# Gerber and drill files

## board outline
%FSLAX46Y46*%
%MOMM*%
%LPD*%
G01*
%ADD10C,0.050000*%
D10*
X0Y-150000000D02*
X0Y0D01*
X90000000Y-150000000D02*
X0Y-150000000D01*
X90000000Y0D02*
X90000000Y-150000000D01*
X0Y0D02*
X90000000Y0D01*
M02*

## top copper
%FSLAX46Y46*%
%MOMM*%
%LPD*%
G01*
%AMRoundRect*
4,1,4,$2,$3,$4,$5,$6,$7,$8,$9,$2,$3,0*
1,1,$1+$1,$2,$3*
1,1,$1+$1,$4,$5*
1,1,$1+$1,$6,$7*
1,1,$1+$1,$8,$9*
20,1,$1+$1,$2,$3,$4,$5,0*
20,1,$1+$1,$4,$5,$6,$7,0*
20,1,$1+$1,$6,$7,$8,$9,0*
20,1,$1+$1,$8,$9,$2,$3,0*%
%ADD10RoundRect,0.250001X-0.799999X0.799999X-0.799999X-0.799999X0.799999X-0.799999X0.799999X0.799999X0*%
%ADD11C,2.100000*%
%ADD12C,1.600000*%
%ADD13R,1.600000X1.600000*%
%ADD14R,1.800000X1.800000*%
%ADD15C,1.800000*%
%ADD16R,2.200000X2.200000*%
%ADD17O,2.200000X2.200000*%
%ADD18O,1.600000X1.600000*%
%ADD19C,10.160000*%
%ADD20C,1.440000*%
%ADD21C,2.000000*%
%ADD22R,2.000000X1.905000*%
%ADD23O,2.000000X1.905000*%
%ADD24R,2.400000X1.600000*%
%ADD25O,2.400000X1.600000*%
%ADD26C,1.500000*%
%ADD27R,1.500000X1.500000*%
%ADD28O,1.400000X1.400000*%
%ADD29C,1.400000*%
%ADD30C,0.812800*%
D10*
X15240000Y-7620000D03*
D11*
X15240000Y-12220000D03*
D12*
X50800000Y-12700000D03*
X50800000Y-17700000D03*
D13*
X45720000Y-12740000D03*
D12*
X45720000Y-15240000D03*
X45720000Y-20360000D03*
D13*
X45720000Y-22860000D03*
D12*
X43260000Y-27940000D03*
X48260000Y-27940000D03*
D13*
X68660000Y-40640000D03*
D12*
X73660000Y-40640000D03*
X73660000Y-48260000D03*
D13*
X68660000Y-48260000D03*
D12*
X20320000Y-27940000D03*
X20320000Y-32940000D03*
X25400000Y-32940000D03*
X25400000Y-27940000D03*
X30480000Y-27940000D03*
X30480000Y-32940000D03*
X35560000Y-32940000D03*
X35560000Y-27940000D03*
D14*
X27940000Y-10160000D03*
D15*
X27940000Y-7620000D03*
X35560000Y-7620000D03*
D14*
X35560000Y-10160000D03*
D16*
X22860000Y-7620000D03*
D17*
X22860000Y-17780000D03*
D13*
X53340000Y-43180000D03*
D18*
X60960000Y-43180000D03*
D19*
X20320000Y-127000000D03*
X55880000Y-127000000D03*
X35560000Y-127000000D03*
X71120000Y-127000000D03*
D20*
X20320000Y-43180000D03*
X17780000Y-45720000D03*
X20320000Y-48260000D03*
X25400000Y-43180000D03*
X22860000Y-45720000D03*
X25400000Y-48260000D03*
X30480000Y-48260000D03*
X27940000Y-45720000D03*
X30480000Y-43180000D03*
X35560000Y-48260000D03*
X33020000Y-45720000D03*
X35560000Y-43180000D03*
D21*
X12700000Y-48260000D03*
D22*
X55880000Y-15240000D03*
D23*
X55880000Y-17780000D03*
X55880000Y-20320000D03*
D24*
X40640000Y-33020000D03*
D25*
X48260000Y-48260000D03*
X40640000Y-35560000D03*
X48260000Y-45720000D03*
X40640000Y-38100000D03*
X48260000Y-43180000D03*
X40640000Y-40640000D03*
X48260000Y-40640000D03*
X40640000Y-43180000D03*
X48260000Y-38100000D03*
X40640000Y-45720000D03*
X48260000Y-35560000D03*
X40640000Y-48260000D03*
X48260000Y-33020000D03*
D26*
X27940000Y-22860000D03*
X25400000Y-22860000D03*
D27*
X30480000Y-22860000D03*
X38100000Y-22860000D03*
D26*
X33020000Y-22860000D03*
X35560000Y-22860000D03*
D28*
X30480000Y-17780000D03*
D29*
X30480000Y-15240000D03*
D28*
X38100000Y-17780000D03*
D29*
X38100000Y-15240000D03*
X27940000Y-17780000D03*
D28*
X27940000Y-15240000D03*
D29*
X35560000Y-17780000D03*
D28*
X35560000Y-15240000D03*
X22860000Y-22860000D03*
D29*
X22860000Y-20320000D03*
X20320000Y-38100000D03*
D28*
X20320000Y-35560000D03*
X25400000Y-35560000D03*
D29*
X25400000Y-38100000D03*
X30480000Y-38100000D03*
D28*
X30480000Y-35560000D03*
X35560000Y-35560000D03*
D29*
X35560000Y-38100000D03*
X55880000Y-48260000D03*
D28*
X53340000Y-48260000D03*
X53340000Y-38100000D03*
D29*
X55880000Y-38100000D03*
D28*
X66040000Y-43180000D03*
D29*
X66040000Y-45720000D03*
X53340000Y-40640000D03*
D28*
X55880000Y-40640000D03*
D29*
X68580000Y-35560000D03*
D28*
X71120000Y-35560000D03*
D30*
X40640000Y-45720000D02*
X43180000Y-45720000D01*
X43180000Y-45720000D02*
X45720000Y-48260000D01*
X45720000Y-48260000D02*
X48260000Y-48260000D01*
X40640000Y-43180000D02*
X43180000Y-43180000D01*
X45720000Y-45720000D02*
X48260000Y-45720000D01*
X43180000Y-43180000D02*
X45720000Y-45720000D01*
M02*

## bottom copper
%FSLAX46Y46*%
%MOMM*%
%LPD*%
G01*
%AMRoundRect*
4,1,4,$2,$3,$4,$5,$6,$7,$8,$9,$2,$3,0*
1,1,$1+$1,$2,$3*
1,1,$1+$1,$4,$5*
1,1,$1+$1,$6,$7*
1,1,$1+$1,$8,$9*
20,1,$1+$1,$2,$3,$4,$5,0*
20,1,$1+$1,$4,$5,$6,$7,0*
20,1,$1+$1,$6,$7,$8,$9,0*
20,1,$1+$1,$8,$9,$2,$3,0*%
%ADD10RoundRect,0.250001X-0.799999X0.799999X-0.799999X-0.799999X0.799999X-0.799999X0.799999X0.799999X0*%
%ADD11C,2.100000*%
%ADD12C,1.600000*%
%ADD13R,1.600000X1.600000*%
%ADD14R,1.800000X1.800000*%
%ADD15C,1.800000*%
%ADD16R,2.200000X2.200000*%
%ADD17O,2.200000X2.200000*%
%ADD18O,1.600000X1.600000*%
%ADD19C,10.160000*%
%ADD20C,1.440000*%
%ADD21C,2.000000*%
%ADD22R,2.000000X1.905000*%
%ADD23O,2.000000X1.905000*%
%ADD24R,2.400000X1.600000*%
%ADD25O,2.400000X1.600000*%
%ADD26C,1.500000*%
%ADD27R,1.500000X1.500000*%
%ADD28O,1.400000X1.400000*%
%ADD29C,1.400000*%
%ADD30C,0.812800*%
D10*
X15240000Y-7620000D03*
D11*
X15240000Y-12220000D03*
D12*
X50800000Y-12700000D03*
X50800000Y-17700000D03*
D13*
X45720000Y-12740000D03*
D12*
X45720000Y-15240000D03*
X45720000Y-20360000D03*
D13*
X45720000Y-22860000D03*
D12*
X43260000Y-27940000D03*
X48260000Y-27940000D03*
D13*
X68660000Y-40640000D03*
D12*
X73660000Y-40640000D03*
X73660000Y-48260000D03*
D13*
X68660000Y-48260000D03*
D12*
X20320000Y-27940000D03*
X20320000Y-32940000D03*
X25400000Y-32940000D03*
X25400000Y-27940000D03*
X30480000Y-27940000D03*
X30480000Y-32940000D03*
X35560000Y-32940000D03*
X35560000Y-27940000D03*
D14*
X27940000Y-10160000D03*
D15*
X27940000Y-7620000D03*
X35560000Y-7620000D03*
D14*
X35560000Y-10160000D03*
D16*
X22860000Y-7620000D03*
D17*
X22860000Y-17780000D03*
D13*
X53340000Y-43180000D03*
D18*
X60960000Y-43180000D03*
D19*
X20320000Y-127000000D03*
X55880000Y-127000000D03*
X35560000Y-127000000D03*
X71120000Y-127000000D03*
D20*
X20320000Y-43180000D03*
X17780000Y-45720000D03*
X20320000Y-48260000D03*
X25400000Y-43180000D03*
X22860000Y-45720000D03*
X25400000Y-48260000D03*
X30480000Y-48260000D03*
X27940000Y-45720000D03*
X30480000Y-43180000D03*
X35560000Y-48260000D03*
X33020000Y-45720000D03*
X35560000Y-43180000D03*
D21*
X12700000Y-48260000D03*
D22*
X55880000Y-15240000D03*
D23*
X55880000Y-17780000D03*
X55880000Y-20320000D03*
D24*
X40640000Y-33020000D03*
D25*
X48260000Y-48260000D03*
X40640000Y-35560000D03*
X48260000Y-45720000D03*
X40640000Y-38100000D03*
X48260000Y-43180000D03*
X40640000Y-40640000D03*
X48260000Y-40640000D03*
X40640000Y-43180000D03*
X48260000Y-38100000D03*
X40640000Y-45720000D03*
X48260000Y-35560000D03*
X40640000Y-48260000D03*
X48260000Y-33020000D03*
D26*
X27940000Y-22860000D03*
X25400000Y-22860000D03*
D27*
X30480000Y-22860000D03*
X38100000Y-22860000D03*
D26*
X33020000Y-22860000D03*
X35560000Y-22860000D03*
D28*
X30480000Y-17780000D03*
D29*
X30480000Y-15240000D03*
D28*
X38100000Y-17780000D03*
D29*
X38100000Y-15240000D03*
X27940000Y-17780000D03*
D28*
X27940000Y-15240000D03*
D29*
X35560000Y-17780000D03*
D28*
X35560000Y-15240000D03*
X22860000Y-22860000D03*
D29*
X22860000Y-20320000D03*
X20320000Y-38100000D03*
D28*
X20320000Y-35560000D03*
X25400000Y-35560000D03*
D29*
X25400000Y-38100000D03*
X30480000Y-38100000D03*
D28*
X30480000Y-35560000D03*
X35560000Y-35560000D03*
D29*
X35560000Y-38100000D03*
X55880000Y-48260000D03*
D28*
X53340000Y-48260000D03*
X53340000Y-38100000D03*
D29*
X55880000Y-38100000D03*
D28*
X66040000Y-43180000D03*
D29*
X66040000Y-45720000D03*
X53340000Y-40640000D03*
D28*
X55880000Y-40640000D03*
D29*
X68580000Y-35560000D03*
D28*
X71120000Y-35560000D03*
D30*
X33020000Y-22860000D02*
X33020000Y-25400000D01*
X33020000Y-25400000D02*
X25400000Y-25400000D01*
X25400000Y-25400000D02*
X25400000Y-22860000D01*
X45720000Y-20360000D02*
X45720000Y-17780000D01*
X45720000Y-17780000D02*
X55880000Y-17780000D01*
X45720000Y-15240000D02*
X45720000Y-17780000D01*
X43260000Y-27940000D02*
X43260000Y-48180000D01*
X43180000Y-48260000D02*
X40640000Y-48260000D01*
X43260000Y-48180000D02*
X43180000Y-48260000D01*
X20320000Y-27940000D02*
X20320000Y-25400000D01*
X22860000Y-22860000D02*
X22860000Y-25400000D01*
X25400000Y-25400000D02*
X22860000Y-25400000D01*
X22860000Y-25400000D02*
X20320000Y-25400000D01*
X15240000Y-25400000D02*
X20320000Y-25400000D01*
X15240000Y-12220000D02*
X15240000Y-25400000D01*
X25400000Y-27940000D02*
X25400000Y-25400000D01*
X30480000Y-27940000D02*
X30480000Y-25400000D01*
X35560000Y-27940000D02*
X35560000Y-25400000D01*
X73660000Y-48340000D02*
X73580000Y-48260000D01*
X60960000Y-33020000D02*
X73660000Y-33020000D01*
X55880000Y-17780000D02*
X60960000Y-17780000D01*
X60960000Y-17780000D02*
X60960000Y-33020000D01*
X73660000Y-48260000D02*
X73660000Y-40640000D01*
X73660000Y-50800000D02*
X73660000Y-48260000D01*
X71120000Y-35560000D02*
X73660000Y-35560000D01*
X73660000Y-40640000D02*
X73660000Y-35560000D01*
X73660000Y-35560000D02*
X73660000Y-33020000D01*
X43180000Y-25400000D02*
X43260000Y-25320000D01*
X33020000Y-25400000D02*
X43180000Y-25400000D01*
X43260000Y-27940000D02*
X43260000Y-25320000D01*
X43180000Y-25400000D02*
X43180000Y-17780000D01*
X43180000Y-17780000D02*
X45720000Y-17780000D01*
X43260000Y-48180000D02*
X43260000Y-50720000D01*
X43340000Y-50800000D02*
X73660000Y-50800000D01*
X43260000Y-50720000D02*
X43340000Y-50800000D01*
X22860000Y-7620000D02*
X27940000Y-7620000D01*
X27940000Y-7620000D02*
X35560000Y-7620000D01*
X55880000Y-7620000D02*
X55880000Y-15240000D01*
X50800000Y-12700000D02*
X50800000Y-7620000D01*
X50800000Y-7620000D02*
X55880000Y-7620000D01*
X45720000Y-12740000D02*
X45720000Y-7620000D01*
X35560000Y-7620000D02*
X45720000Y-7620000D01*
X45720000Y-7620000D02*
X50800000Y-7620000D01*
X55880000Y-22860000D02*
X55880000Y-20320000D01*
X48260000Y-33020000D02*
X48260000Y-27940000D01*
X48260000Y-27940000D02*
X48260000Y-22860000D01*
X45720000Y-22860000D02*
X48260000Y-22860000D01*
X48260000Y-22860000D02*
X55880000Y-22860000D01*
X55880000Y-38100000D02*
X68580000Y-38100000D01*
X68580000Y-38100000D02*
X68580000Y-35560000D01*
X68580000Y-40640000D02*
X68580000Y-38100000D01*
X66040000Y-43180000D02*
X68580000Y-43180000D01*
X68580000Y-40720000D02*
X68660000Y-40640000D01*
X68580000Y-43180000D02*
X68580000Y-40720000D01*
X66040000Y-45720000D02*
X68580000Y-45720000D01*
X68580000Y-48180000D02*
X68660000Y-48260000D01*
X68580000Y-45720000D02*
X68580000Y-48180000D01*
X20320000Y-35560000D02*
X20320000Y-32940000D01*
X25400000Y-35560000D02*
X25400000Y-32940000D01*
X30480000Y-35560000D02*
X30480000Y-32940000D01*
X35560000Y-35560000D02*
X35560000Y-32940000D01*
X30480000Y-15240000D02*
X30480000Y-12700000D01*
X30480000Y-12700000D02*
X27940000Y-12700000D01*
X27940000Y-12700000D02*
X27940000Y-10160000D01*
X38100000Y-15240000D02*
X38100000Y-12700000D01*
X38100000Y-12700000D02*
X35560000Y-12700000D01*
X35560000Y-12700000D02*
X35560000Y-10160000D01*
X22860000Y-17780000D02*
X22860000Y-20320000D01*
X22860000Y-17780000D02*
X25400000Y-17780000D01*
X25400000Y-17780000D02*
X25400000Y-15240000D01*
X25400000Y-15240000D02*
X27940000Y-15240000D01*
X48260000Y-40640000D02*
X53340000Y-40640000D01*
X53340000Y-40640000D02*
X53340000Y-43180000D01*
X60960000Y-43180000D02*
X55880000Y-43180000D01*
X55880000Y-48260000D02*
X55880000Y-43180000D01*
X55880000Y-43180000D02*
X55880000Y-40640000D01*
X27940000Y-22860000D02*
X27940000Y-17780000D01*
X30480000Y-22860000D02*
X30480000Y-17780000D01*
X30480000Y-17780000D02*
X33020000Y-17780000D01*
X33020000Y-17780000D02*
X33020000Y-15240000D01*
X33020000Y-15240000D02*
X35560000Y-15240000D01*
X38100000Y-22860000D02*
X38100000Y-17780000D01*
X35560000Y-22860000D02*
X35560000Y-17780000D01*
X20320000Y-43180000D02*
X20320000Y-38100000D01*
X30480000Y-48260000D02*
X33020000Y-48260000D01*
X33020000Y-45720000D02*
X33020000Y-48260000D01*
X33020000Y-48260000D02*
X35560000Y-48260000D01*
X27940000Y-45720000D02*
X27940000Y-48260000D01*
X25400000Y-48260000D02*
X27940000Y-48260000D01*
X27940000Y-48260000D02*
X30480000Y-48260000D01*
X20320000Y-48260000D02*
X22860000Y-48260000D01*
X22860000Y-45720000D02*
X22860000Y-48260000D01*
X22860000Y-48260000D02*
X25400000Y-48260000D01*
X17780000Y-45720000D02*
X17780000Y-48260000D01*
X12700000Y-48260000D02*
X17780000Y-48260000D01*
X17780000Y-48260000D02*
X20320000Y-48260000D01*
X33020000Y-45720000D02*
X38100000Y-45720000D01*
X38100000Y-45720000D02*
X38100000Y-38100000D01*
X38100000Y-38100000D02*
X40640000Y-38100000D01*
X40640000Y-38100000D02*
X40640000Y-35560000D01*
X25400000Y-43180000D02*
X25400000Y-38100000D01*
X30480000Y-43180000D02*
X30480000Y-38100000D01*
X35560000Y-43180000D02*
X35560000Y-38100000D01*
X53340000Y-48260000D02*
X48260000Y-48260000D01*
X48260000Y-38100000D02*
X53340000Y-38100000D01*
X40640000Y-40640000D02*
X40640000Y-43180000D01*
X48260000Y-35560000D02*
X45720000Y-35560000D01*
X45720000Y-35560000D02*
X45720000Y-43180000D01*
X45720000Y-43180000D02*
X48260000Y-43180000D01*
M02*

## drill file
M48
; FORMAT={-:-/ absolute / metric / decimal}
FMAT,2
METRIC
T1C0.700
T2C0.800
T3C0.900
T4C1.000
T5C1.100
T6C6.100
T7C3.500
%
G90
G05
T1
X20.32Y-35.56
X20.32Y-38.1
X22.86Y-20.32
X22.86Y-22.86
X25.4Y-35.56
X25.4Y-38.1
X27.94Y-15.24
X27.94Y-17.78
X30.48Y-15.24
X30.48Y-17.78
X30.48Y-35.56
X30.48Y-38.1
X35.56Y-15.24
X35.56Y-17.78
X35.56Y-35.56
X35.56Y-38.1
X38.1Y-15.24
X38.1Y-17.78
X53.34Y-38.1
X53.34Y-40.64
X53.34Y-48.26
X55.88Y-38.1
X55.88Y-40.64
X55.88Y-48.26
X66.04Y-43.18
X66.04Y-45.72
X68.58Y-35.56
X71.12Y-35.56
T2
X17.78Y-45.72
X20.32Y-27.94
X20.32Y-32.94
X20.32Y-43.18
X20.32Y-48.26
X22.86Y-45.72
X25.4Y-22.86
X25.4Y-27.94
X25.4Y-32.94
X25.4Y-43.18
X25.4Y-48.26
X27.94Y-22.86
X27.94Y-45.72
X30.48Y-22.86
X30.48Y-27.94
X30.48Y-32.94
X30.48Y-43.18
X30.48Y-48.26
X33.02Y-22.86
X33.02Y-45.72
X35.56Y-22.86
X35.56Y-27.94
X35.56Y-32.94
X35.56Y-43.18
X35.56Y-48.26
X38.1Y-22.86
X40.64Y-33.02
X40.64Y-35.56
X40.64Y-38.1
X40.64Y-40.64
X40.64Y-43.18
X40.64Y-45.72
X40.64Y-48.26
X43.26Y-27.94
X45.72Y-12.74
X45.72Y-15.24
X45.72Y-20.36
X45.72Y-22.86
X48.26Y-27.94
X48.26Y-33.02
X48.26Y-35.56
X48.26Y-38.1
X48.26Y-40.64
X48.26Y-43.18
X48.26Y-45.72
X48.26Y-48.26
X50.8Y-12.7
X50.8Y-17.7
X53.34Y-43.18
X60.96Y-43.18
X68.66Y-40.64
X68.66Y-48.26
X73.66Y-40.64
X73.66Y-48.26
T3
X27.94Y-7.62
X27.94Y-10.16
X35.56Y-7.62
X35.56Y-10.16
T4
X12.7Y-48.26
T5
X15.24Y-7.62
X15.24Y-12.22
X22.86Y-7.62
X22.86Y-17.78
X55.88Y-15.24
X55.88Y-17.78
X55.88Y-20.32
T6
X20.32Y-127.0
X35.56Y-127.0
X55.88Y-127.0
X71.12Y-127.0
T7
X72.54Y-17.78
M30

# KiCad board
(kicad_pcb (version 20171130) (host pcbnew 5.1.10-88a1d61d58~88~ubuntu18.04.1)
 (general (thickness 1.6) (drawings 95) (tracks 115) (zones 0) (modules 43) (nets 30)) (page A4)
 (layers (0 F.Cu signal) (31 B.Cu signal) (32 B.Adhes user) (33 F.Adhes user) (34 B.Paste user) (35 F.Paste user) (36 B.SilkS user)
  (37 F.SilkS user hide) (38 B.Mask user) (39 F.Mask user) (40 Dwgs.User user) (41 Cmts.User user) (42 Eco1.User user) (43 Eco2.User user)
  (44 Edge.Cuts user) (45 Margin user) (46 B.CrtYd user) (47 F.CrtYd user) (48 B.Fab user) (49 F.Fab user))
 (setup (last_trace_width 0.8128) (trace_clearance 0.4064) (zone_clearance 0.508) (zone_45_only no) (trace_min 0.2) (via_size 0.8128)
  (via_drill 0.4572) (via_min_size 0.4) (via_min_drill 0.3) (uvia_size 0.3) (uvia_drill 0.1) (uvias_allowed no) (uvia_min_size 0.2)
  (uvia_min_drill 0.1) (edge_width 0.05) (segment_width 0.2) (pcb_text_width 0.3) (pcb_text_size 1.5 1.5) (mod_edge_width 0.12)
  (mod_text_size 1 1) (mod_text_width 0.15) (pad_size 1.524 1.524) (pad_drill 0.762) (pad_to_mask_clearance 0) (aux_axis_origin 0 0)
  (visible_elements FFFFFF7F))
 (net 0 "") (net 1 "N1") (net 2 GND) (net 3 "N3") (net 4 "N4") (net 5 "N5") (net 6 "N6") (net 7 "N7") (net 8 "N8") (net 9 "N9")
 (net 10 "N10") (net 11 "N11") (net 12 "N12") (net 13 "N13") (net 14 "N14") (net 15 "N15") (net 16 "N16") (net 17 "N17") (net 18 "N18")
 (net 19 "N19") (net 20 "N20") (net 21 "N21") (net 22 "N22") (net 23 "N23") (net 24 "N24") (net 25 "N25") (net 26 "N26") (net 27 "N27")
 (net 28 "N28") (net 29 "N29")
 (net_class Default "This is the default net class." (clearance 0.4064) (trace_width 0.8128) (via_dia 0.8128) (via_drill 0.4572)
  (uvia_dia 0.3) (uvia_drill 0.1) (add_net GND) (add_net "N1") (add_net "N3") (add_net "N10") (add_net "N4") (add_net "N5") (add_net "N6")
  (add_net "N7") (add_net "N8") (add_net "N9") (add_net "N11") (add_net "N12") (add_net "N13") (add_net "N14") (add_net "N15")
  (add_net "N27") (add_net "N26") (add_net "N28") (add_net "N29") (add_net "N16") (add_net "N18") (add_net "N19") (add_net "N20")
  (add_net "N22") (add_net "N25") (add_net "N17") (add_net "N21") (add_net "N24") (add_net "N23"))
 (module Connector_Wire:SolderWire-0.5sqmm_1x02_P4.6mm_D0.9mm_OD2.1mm (layer F.Cu) (at 15.24 7.62 270)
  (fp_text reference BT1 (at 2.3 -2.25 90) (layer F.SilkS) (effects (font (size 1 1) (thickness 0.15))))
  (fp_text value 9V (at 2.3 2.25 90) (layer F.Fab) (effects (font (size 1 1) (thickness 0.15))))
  (pad 1 thru_hole roundrect (at 0 0 270) (size 2.1 2.1) (drill 1.1) (layers *.Cu *.Mask) (roundrect_rratio 0.119048) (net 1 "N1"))
  (pad 2 thru_hole circle (at 4.6 0 270) (size 2.1 2.1) (drill 1.1) (layers *.Cu *.Mask) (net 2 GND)))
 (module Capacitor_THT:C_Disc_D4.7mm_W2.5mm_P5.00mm (layer F.Cu) (at 50.8 12.7 270)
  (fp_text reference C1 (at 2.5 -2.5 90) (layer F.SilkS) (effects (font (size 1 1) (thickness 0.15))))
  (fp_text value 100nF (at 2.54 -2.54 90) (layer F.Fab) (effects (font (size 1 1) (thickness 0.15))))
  (pad 1 thru_hole circle (at 0 0 270) (size 1.6 1.6) (drill 0.8) (layers *.Cu *.Mask) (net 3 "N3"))
  (pad 2 thru_hole circle (at 5 0 270) (size 1.6 1.6) (drill 0.8) (layers *.Cu *.Mask) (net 2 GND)))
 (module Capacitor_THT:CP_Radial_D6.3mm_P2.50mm (layer F.Cu) (at 45.72 12.74 270)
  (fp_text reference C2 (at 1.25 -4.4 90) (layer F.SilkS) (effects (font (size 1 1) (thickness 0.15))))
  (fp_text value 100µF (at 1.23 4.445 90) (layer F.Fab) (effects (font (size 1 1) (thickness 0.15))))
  (pad 1 thru_hole rect (at 0 0 270) (size 1.6 1.6) (drill 0.8) (layers *.Cu *.Mask) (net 3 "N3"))
  (pad 2 thru_hole circle (at 2.5 0 270) (size 1.6 1.6) (drill 0.8) (layers *.Cu *.Mask) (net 2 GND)))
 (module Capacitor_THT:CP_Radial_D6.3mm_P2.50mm (layer F.Cu) (at 45.72 22.86 90)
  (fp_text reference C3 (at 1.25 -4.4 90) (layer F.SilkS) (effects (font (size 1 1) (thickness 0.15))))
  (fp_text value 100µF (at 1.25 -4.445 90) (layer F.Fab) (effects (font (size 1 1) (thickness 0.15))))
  (pad 2 thru_hole circle (at 2.5 0 90) (size 1.6 1.6) (drill 0.8) (layers *.Cu *.Mask) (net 2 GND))
  (pad 1 thru_hole rect (at 0 0 90) (size 1.6 1.6) (drill 0.8) (layers *.Cu *.Mask) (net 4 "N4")))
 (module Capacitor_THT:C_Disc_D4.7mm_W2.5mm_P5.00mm (layer F.Cu) (at 48.26 27.94 180)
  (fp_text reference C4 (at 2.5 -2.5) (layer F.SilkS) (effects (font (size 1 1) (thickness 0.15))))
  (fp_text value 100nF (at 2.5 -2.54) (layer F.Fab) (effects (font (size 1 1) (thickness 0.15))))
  (pad 2 thru_hole circle (at 5 0 180) (size 1.6 1.6) (drill 0.8) (layers *.Cu *.Mask) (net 2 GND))
  (pad 1 thru_hole circle (at 0 0 180) (size 1.6 1.6) (drill 0.8) (layers *.Cu *.Mask) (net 4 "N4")))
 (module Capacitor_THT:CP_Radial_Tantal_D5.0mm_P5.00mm (layer F.Cu) (at 68.66 40.64)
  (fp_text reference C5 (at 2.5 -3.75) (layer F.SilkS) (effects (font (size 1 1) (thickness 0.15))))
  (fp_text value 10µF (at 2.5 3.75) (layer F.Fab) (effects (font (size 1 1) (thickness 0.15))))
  (pad 1 thru_hole rect (at 0 0) (size 1.6 1.6) (drill 0.8) (layers *.Cu *.Mask) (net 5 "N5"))
  (pad 2 thru_hole circle (at 5 0) (size 1.6 1.6) (drill 0.8) (layers *.Cu *.Mask) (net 2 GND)))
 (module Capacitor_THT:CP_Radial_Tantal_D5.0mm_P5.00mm (layer F.Cu) (at 68.66 48.26)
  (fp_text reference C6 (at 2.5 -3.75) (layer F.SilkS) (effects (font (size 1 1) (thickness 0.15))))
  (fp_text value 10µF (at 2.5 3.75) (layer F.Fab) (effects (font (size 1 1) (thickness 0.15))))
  (pad 2 thru_hole circle (at 5 0) (size 1.6 1.6) (drill 0.8) (layers *.Cu *.Mask) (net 2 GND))
  (pad 1 thru_hole rect (at 0 0) (size 1.6 1.6) (drill 0.8) (layers *.Cu *.Mask) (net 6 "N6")))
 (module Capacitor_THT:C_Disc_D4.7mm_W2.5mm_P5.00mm (layer F.Cu) (at 20.32 32.94 90)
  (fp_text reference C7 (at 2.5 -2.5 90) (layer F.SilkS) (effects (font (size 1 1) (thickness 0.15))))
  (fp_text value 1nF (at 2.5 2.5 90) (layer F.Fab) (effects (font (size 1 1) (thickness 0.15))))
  (pad 2 thru_hole circle (at 5 0 90) (size 1.6 1.6) (drill 0.8) (layers *.Cu *.Mask) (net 2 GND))
  (pad 1 thru_hole circle (at 0 0 90) (size 1.6 1.6) (drill 0.8) (layers *.Cu *.Mask) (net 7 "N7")))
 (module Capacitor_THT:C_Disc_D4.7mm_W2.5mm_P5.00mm (layer F.Cu) (at 25.4 32.94 90)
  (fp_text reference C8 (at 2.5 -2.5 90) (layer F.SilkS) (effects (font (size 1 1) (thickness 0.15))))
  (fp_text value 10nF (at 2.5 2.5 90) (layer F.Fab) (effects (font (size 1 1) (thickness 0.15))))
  (pad 1 thru_hole circle (at 0 0 90) (size 1.6 1.6) (drill 0.8) (layers *.Cu *.Mask) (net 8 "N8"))
  (pad 2 thru_hole circle (at 5 0 90) (size 1.6 1.6) (drill 0.8) (layers *.Cu *.Mask) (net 2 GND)))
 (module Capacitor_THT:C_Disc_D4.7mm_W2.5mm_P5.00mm (layer F.Cu) (at 30.48 32.94 90)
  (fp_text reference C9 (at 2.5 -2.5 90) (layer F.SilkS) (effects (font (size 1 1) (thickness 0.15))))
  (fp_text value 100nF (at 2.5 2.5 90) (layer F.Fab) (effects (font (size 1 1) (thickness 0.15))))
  (pad 2 thru_hole circle (at 5 0 90) (size 1.6 1.6) (drill 0.8) (layers *.Cu *.Mask) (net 2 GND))
  (pad 1 thru_hole circle (at 0 0 90) (size 1.6 1.6) (drill 0.8) (layers *.Cu *.Mask) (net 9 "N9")))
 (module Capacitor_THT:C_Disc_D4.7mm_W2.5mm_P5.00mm (layer F.Cu) (at 35.56 32.94 90)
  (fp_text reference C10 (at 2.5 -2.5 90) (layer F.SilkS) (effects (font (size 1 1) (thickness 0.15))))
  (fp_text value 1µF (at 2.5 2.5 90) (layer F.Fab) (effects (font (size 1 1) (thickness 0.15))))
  (pad 1 thru_hole circle (at 0 0 90) (size 1.6 1.6) (drill 0.8) (layers *.Cu *.Mask) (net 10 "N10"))
  (pad 2 thru_hole circle (at 5 0 90) (size 1.6 1.6) (drill 0.8) (layers *.Cu *.Mask) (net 2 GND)))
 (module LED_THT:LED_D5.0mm (layer F.Cu) (at 27.94 10.16 90)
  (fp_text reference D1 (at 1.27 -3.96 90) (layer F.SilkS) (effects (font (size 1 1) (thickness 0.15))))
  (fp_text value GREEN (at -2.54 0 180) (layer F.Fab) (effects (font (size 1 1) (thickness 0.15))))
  (pad 1 thru_hole rect (at 0 0 90) (size 1.8 1.8) (drill 0.9) (layers *.Cu *.Mask) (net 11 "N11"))
  (pad 2 thru_hole circle (at 2.54 0 90) (size 1.8 1.8) (drill 0.9) (layers *.Cu *.Mask) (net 3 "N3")))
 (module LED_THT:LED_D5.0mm (layer F.Cu) (at 35.56 10.16 90)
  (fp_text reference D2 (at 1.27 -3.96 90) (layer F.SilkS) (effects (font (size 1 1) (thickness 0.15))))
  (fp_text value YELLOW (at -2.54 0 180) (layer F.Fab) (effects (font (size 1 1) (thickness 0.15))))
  (pad 2 thru_hole circle (at 2.54 0 90) (size 1.8 1.8) (drill 0.9) (layers *.Cu *.Mask) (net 3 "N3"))
  (pad 1 thru_hole rect (at 0 0 90) (size 1.8 1.8) (drill 0.9) (layers *.Cu *.Mask) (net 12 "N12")))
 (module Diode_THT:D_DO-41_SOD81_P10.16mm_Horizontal (layer F.Cu) (at 22.86 7.62 270)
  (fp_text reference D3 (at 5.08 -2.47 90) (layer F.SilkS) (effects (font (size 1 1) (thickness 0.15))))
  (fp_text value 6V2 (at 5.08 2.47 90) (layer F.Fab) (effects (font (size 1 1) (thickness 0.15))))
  (pad 1 thru_hole rect (at 0 0 270) (size 2.2 2.2) (drill 1.1) (layers *.Cu *.Mask) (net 3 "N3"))
  (pad 2 thru_hole oval (at 10.16 0 270) (size 2.2 2.2) (drill 1.1) (layers *.Cu *.Mask) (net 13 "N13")))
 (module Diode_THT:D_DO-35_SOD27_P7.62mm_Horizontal (layer F.Cu) (at 53.34 43.18)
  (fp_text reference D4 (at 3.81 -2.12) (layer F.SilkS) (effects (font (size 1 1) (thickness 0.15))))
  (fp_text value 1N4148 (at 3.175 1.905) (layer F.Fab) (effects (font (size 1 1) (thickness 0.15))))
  (pad 1 thru_hole rect (at 0 0) (size 1.6 1.6) (drill 0.8) (layers *.Cu *.Mask) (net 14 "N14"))
  (pad 2 thru_hole oval (at 7.62 0) (size 1.6 1.6) (drill 0.8) (layers *.Cu *.Mask) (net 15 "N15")))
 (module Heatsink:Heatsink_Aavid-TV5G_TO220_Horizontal (layer F.Cu) (at 72.39 17.78 270)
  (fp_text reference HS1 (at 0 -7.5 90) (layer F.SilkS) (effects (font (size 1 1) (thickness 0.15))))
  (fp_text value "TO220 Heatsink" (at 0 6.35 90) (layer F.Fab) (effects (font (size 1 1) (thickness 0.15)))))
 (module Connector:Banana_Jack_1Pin (layer F.Cu) (at 20.32 127)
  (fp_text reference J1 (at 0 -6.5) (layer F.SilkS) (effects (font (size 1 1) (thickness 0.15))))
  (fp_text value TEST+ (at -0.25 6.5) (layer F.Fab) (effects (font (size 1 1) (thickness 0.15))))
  (pad 1 thru_hole circle (at 0 0) (size 10.16 10.16) (drill 6.1) (layers *.Cu *.Mask) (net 15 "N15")))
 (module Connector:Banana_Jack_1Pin (layer F.Cu) (at 55.88 127)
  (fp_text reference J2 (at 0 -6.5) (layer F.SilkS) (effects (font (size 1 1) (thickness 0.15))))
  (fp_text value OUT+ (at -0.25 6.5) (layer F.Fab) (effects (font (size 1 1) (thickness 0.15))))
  (pad 1 thru_hole circle (at 0 0) (size 10.16 10.16) (drill 6.1) (layers *.Cu *.Mask) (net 6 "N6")))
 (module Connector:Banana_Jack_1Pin (layer F.Cu) (at 35.56 127)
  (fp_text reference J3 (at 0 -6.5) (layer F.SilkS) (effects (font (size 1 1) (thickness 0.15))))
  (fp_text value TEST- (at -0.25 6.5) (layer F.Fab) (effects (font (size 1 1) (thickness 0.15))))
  (pad 1 thru_hole circle (at 0 0) (size 10.16 10.16) (drill 6.1) (layers *.Cu *.Mask) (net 2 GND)))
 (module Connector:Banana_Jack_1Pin (layer F.Cu) (at 71.12 127)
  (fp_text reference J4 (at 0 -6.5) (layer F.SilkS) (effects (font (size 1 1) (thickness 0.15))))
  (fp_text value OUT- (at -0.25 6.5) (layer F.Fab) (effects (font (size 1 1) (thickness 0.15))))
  (pad 1 thru_hole circle (at 0 0) (size 10.16 10.16) (drill 6.1) (layers *.Cu *.Mask) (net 2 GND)))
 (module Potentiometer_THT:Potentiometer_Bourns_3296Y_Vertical (layer F.Cu) (at 20.32 48.26 270)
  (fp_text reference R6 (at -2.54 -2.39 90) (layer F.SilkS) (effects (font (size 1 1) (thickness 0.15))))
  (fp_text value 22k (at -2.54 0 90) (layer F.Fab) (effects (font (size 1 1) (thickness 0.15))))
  (pad 3 thru_hole circle (at -5.08 0 270) (size 1.44 1.44) (drill 0.8) (layers *.Cu *.Mask) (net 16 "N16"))
  (pad 2 thru_hole circle (at -2.54 2.54 270) (size 1.44 1.44) (drill 0.8) (layers *.Cu *.Mask) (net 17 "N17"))
  (pad 1 thru_hole circle (at 0 0 270) (size 1.44 1.44) (drill 0.8) (layers *.Cu *.Mask) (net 17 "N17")))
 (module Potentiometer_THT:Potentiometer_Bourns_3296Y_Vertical (layer F.Cu) (at 25.4 48.26 270)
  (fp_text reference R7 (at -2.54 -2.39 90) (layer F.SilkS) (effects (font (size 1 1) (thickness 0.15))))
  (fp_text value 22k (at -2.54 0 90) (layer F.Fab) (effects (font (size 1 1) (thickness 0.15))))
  (pad 3 thru_hole circle (at -5.08 0 270) (size 1.44 1.44) (drill 0.8) (layers *.Cu *.Mask) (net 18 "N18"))
  (pad 2 thru_hole circle (at -2.54 2.54 270) (size 1.44 1.44) (drill 0.8) (layers *.Cu *.Mask) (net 17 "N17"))
  (pad 1 thru_hole circle (at 0 0 270) (size 1.44 1.44) (drill 0.8) (layers *.Cu *.Mask) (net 17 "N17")))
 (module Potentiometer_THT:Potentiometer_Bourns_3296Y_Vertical (layer F.Cu) (at 30.48 48.26 270)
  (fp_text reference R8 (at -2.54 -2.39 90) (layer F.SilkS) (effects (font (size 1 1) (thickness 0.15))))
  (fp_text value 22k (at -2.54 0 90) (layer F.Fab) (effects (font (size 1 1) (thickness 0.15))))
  (pad 1 thru_hole circle (at 0 0 270) (size 1.44 1.44) (drill 0.8) (layers *.Cu *.Mask) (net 17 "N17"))
  (pad 2 thru_hole circle (at -2.54 2.54 270) (size 1.44 1.44) (drill 0.8) (layers *.Cu *.Mask) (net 17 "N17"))
  (pad 3 thru_hole circle (at -5.08 0 270) (size 1.44 1.44) (drill 0.8) (layers *.Cu *.Mask) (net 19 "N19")))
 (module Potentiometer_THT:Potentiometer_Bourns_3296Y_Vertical (layer F.Cu) (at 35.56 48.26 270)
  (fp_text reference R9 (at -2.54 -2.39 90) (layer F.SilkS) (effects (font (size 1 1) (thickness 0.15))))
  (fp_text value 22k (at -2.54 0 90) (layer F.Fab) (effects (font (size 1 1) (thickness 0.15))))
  (pad 1 thru_hole circle (at 0 0 270) (size 1.44 1.44) (drill 0.8) (layers *.Cu *.Mask) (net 17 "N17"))
  (pad 2 thru_hole circle (at -2.54 2.54 270) (size 1.44 1.44) (drill 0.8) (layers *.Cu *.Mask) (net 17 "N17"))
  (pad 3 thru_hole circle (at -5.08 0 270) (size 1.44 1.44) (drill 0.8) (layers *.Cu *.Mask) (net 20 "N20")))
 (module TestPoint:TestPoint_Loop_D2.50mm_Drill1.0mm (layer F.Cu) (at 12.7 48.26)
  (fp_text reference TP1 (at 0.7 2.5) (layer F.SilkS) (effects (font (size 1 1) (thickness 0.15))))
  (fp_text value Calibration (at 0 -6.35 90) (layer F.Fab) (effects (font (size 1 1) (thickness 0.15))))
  (pad 1 thru_hole circle (at 0 0) (size 2 2) (drill 1) (layers *.Cu *.Mask) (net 17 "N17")))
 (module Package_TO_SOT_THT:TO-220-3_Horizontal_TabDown (layer F.Cu) (at 55.88 15.24 270)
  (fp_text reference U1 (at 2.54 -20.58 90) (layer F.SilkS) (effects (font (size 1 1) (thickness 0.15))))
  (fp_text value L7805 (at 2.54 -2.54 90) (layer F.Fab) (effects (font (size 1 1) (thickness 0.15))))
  (pad "" np_thru_hole oval (at 2.54 -16.66 270) (size 3.5 3.5) (drill 3.5) (layers *.Cu *.Mask))
  (pad 1 thru_hole rect (at 0 0 270) (size 1.905 2) (drill 1.1) (layers *.Cu *.Mask) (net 3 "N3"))
  (pad 2 thru_hole oval (at 2.54 0 270) (size 1.905 2) (drill 1.1) (layers *.Cu *.Mask) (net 2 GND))
  (pad 3 thru_hole oval (at 5.08 0 270) (size 1.905 2) (drill 1.1) (layers *.Cu *.Mask) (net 4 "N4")))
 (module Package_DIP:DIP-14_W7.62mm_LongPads (layer F.Cu) (at 40.64 33.02)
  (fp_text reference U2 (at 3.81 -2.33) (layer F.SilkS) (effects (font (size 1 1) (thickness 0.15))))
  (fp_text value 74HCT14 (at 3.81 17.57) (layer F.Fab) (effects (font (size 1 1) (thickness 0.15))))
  (pad 1 thru_hole rect (at 0 0) (size 2.4 1.6) (drill 0.8) (layers *.Cu *.Mask) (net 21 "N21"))
  (pad 8 thru_hole oval (at 7.62 15.24) (size 2.4 1.6) (drill 0.8) (layers *.Cu *.Mask) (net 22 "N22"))
  (pad 2 thru_hole oval (at 0 2.54) (size 2.4 1.6) (drill 0.8) (layers *.Cu *.Mask) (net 17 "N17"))
  (pad 9 thru_hole oval (at 7.62 12.7) (size 2.4 1.6) (drill 0.8) (layers *.Cu *.Mask) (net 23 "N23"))
  (pad 3 thru_hole oval (at 0 5.08) (size 2.4 1.6) (drill 0.8) (layers *.Cu *.Mask) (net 17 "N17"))
  (pad 10 thru_hole oval (at 7.62 10.16) (size 2.4 1.6) (drill 0.8) (layers *.Cu *.Mask) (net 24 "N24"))
  (pad 4 thru_hole oval (at 0 7.62) (size 2.4 1.6) (drill 0.8) (layers *.Cu *.Mask) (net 23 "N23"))
  (pad 11 thru_hole oval (at 7.62 7.62) (size 2.4 1.6) (drill 0.8) (layers *.Cu *.Mask) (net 14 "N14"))
  (pad 5 thru_hole oval (at 0 10.16) (size 2.4 1.6) (drill 0.8) (layers *.Cu *.Mask) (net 23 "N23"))
  (pad 12 thru_hole oval (at 7.62 5.08) (size 2.4 1.6) (drill 0.8) (layers *.Cu *.Mask) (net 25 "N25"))
  (pad 6 thru_hole oval (at 0 12.7) (size 2.4 1.6) (drill 0.8) (layers *.Cu *.Mask) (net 22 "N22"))
  (pad 13 thru_hole oval (at 7.62 2.54) (size 2.4 1.6) (drill 0.8) (layers *.Cu *.Mask) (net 24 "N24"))
  (pad 7 thru_hole oval (at 0 15.24) (size 2.4 1.6) (drill 0.8) (layers *.Cu *.Mask) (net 2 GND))
  (pad 14 thru_hole oval (at 7.62 0) (size 2.4 1.6) (drill 0.8) (layers *.Cu *.Mask) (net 4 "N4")))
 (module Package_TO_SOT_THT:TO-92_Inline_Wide (layer F.Cu) (at 30.48 22.86 180)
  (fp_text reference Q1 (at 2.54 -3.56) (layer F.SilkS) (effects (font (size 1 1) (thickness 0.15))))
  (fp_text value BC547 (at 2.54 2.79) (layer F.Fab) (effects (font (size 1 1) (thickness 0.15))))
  (pad 2 thru_hole circle (at 2.54 0 180) (size 1.5 1.5) (drill 0.8) (layers *.Cu *.Mask) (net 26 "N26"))
  (pad 3 thru_hole circle (at 5.08 0 180) (size 1.5 1.5) (drill 0.8) (layers *.Cu *.Mask) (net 2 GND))
  (pad 1 thru_hole rect (at 0 0 180) (size 1.5 1.5) (drill 0.8) (layers *.Cu *.Mask) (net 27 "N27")))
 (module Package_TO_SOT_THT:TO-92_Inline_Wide (layer F.Cu) (at 38.1 22.86 180)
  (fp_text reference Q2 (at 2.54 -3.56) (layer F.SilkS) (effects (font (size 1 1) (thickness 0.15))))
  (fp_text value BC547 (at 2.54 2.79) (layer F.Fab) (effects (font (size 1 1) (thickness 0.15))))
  (pad 1 thru_hole rect (at 0 0 180) (size 1.5 1.5) (drill 0.8) (layers *.Cu *.Mask) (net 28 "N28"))
  (pad 3 thru_hole circle (at 5.08 0 180) (size 1.5 1.5) (drill 0.8) (layers *.Cu *.Mask) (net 2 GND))
  (pad 2 thru_hole circle (at 2.54 0 180) (size 1.5 1.5) (drill 0.8) (layers *.Cu *.Mask) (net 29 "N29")))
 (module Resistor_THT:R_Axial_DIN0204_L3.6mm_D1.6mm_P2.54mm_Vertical (layer F.Cu) (at 30.48 15.24 270)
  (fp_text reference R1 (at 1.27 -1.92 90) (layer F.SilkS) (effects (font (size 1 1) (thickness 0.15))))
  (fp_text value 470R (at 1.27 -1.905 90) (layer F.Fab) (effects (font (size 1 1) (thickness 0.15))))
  (pad 2 thru_hole oval (at 2.54 0 270) (size 1.4 1.4) (drill 0.7) (layers *.Cu *.Mask) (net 27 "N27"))
  (pad 1 thru_hole circle (at 0 0 270) (size 1.4 1.4) (drill 0.7) (layers *.Cu *.Mask) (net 11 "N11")))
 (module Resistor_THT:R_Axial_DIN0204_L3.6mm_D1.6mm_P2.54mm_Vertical (layer F.Cu) (at 38.1 15.24 270)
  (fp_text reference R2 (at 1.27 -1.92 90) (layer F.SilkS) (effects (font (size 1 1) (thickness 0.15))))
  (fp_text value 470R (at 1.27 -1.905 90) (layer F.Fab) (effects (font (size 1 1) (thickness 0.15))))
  (pad 2 thru_hole oval (at 2.54 0 270) (size 1.4 1.4) (drill 0.7) (layers *.Cu *.Mask) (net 28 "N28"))
  (pad 1 thru_hole circle (at 0 0 270) (size 1.4 1.4) (drill 0.7) (layers *.Cu *.Mask) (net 12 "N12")))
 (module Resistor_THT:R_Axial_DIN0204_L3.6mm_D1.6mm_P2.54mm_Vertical (layer F.Cu) (at 27.94 17.78 90)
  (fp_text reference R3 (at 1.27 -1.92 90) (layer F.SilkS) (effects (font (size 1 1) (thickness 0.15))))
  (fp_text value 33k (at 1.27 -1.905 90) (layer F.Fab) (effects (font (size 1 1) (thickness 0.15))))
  (pad 1 thru_hole circle (at 0 0 90) (size 1.4 1.4) (drill 0.7) (layers *.Cu *.Mask) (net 26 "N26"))
  (pad 2 thru_hole oval (at 2.54 0 90) (size 1.4 1.4) (drill 0.7) (layers *.Cu *.Mask) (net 13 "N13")))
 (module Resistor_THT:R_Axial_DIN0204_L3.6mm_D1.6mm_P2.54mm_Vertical (layer F.Cu) (at 35.56 17.78 90)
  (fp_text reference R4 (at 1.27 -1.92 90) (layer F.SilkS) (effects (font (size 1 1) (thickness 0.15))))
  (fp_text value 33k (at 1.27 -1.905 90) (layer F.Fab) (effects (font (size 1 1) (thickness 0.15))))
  (pad 1 thru_hole circle (at 0 0 90) (size 1.4 1.4) (drill 0.7) (layers *.Cu *.Mask) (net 29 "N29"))
  (pad 2 thru_hole oval (at 2.54 0 90) (size 1.4 1.4) (drill 0.7) (layers *.Cu *.Mask) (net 27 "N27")))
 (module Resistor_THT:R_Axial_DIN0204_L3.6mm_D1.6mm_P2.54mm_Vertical (layer F.Cu) (at 22.86 20.32 270)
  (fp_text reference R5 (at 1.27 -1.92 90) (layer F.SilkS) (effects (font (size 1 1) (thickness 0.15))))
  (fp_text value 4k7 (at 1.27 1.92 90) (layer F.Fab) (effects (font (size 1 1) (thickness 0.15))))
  (pad 2 thru_hole oval (at 2.54 0 270) (size 1.4 1.4) (drill 0.7) (layers *.Cu *.Mask) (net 2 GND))
  (pad 1 thru_hole circle (at 0 0 270) (size 1.4 1.4) (drill 0.7) (layers *.Cu *.Mask) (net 13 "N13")))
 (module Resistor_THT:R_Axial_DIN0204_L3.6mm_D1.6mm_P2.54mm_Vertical (layer F.Cu) (at 20.32 38.1 90)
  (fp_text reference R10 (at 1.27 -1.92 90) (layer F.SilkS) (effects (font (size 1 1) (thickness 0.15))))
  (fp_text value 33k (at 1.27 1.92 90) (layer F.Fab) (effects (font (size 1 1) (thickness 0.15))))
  (pad 1 thru_hole circle (at 0 0 90) (size 1.4 1.4) (drill 0.7) (layers *.Cu *.Mask) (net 16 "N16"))
  (pad 2 thru_hole oval (at 2.54 0 90) (size 1.4 1.4) (drill 0.7) (layers *.Cu *.Mask) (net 7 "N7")))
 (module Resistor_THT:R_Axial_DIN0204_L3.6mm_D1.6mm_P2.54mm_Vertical (layer F.Cu) (at 25.4 38.1 90)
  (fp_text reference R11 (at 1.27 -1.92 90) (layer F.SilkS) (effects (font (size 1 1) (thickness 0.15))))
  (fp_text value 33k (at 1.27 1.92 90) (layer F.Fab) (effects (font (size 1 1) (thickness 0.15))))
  (pad 2 thru_hole oval (at 2.54 0 90) (size 1.4 1.4) (drill 0.7) (layers *.Cu *.Mask) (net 8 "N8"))
  (pad 1 thru_hole circle (at 0 0 90) (size 1.4 1.4) (drill 0.7) (layers *.Cu *.Mask) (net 18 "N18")))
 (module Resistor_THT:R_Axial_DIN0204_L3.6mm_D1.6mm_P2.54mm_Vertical (layer F.Cu) (at 30.48 38.1 90)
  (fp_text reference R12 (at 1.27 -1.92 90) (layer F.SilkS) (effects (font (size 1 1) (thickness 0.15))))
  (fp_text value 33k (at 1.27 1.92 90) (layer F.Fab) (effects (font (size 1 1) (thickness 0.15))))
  (pad 1 thru_hole circle (at 0 0 90) (size 1.4 1.4) (drill 0.7) (layers *.Cu *.Mask) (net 19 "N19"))
  (pad 2 thru_hole oval (at 2.54 0 90) (size 1.4 1.4) (drill 0.7) (layers *.Cu *.Mask) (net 9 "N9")))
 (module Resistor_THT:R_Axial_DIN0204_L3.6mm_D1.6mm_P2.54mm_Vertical (layer F.Cu) (at 35.56 38.1 90)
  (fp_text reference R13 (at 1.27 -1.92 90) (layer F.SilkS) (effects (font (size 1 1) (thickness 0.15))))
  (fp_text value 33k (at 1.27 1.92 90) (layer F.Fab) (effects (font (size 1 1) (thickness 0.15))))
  (pad 2 thru_hole oval (at 2.54 0 90) (size 1.4 1.4) (drill 0.7) (layers *.Cu *.Mask) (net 10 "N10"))
  (pad 1 thru_hole circle (at 0 0 90) (size 1.4 1.4) (drill 0.7) (layers *.Cu *.Mask) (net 20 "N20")))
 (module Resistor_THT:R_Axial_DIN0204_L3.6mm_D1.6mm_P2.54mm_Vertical (layer F.Cu) (at 55.88 48.26 180)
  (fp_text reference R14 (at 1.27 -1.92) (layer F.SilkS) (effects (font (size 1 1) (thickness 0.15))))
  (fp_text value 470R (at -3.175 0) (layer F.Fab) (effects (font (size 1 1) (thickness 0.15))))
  (pad 1 thru_hole circle (at 0 0 180) (size 1.4 1.4) (drill 0.7) (layers *.Cu *.Mask) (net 15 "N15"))
  (pad 2 thru_hole oval (at 2.54 0 180) (size 1.4 1.4) (drill 0.7) (layers *.Cu *.Mask) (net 22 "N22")))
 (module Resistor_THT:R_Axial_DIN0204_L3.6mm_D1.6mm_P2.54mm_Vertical (layer F.Cu) (at 55.88 38.1 180)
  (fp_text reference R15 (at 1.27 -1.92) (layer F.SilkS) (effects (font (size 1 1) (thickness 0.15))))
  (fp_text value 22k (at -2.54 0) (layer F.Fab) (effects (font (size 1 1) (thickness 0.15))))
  (pad 2 thru_hole oval (at 2.54 0 180) (size 1.4 1.4) (drill 0.7) (layers *.Cu *.Mask) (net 25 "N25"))
  (pad 1 thru_hole circle (at 0 0 180) (size 1.4 1.4) (drill 0.7) (layers *.Cu *.Mask) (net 5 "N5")))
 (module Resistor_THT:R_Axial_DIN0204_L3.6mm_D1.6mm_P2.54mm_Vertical (layer F.Cu) (at 66.04 45.72 90)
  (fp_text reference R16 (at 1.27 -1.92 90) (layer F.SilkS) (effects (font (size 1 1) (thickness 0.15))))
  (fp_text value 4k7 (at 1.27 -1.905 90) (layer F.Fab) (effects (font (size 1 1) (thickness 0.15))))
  (pad 2 thru_hole oval (at 2.54 0 90) (size 1.4 1.4) (drill 0.7) (layers *.Cu *.Mask) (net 5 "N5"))
  (pad 1 thru_hole circle (at 0 0 90) (size 1.4 1.4) (drill 0.7) (layers *.Cu *.Mask) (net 6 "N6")))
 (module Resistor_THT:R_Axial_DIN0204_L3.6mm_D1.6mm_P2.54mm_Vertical (layer F.Cu) (at 53.34 40.64)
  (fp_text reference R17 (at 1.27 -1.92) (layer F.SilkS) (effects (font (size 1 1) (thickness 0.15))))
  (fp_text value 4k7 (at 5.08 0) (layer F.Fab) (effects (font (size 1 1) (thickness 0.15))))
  (pad 1 thru_hole circle (at 0 0) (size 1.4 1.4) (drill 0.7) (layers *.Cu *.Mask) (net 14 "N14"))
  (pad 2 thru_hole oval (at 2.54 0) (size 1.4 1.4) (drill 0.7) (layers *.Cu *.Mask) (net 15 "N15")))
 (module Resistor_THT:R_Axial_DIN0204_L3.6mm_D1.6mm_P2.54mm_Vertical (layer F.Cu) (at 68.58 35.56)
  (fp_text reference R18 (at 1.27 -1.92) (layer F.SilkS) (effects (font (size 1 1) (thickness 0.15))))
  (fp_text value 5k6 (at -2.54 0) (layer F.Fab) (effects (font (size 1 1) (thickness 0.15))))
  (pad 1 thru_hole circle (at 0 0) (size 1.4 1.4) (drill 0.7) (layers *.Cu *.Mask) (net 5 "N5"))
  (pad 2 thru_hole oval (at 2.54 0) (size 1.4 1.4) (drill 0.7) (layers *.Cu *.Mask) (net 2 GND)))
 (gr_line (start 0 150) (end 0 0) (layer Edge.Cuts) (width 0.05))
 (gr_line (start 90 150) (end 0 150) (layer Edge.Cuts) (width 0.05))
 (gr_line (start 90 0) (end 90 150) (layer Edge.Cuts) (width 0.05))
 (gr_line (start 0 0) (end 90 0) (layer Edge.Cuts) (width 0.05))
 (segment (start 33.02 22.86) (end 33.02 25.4) (width 0.8128) (layer B.Cu) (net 2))
 (segment (start 33.02 25.4) (end 25.4 25.4) (width 0.8128) (layer B.Cu) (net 2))
 (segment (start 25.4 25.4) (end 25.4 22.86) (width 0.8128) (layer B.Cu) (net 2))
 (segment (start 45.72 20.36) (end 45.72 17.78) (width 0.8128) (layer B.Cu) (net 2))
 (segment (start 45.72 17.78) (end 55.88 17.78) (width 0.8128) (layer B.Cu) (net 2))
 (segment (start 45.72 15.24) (end 45.72 17.78) (width 0.8128) (layer B.Cu) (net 2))
 (segment (start 43.26 27.94) (end 43.26 48.18) (width 0.8128) (layer B.Cu) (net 2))
 (segment (start 43.18 48.26) (end 40.64 48.26) (width 0.8128) (layer B.Cu) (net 2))
 (segment (start 43.26 48.18) (end 43.18 48.26) (width 0.8128) (layer B.Cu) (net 2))
 (segment (start 20.32 27.94) (end 20.32 25.4) (width 0.8128) (layer B.Cu) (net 2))
 (segment (start 22.86 22.86) (end 22.86 25.4) (width 0.8128) (layer B.Cu) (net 2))
 (segment (start 25.4 25.4) (end 22.86 25.4) (width 0.8128) (layer B.Cu) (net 2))
 (segment (start 22.86 25.4) (end 20.32 25.4) (width 0.8128) (layer B.Cu) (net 2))
 (segment (start 15.24 25.4) (end 20.32 25.4) (width 0.8128) (layer B.Cu) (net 2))
 (segment (start 15.24 12.22) (end 15.24 25.4) (width 0.8128) (layer B.Cu) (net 2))
 (segment (start 25.4 27.94) (end 25.4 25.4) (width 0.8128) (layer B.Cu) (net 2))
 (segment (start 30.48 27.94) (end 30.48 25.4) (width 0.8128) (layer B.Cu) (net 2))
 (segment (start 35.56 27.94) (end 35.56 25.4) (width 0.8128) (layer B.Cu) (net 2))
 (segment (start 73.66 48.34) (end 73.58 48.26) (width 0.8128) (layer B.Cu) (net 2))
 (segment (start 60.96 33.02) (end 73.66 33.02) (width 0.8128) (layer B.Cu) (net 2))
 (segment (start 55.88 17.78) (end 60.96 17.78) (width 0.8128) (layer B.Cu) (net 2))
 (segment (start 60.96 17.78) (end 60.96 33.02) (width 0.8128) (layer B.Cu) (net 2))
 (segment (start 73.66 48.26) (end 73.66 40.64) (width 0.8128) (layer B.Cu) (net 2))
 (segment (start 73.66 50.8) (end 73.66 48.26) (width 0.8128) (layer B.Cu) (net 2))
 (segment (start 71.12 35.56) (end 73.66 35.56) (width 0.8128) (layer B.Cu) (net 2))
 (segment (start 73.66 40.64) (end 73.66 35.56) (width 0.8128) (layer B.Cu) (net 2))
 (segment (start 73.66 35.56) (end 73.66 33.02) (width 0.8128) (layer B.Cu) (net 2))
 (segment (start 43.18 25.4) (end 43.26 25.32) (width 0.8128) (layer B.Cu) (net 2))
 (segment (start 33.02 25.4) (end 43.18 25.4) (width 0.8128) (layer B.Cu) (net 2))
 (segment (start 43.26 27.94) (end 43.26 25.32) (width 0.8128) (layer B.Cu) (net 2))
 (segment (start 43.18 25.4) (end 43.18 17.78) (width 0.8128) (layer B.Cu) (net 2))
 (segment (start 43.18 17.78) (end 45.72 17.78) (width 0.8128) (layer B.Cu) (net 2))
 (segment (start 43.26 48.18) (end 43.26 50.72) (width 0.8128) (layer B.Cu) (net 2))
 (segment (start 43.34 50.8) (end 73.66 50.8) (width 0.8128) (layer B.Cu) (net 2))
 (segment (start 43.26 50.72) (end 43.34 50.8) (width 0.8128) (layer B.Cu) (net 2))
 (segment (start 22.86 7.62) (end 27.94 7.62) (width 0.8128) (layer B.Cu) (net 3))
 (segment (start 27.94 7.62) (end 35.56 7.62) (width 0.8128) (layer B.Cu) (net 3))
 (segment (start 55.88 7.62) (end 55.88 15.24) (width 0.8128) (layer B.Cu) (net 3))
 (segment (start 50.8 12.7) (end 50.8 7.62) (width 0.8128) (layer B.Cu) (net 3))
 (segment (start 50.8 7.62) (end 55.88 7.62) (width 0.8128) (layer B.Cu) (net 3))
 (segment (start 45.72 12.74) (end 45.72 7.62) (width 0.8128) (layer B.Cu) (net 3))
 (segment (start 35.56 7.62) (end 45.72 7.62) (width 0.8128) (layer B.Cu) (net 3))
 (segment (start 45.72 7.62) (end 50.8 7.62) (width 0.8128) (layer B.Cu) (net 3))
 (segment (start 55.88 22.86) (end 55.88 20.32) (width 0.8128) (layer B.Cu) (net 4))
 (segment (start 48.26 33.02) (end 48.26 27.94) (width 0.8128) (layer B.Cu) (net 4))
 (segment (start 48.26 27.94) (end 48.26 22.86) (width 0.8128) (layer B.Cu) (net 4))
 (segment (start 45.72 22.86) (end 48.26 22.86) (width 0.8128) (layer B.Cu) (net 4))
 (segment (start 48.26 22.86) (end 55.88 22.86) (width 0.8128) (layer B.Cu) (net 4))
 (segment (start 55.88 38.1) (end 68.58 38.1) (width 0.8128) (layer B.Cu) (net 5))
 (segment (start 68.58 38.1) (end 68.58 35.56) (width 0.8128) (layer B.Cu) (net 5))
 (segment (start 68.58 40.64) (end 68.58 38.1) (width 0.8128) (layer B.Cu) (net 5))
 (segment (start 66.04 43.18) (end 68.58 43.18) (width 0.8128) (layer B.Cu) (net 5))
 (segment (start 68.58 40.72) (end 68.66 40.64) (width 0.8128) (layer B.Cu) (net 5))
 (segment (start 68.58 43.18) (end 68.58 40.72) (width 0.8128) (layer B.Cu) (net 5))
 (segment (start 66.04 45.72) (end 68.58 45.72) (width 0.8128) (layer B.Cu) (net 6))
 (segment (start 68.58 48.18) (end 68.66 48.26) (width 0.8128) (layer B.Cu) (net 6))
 (segment (start 68.58 45.72) (end 68.58 48.18) (width 0.8128) (layer B.Cu) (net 6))
 (segment (start 20.32 35.56) (end 20.32 32.94) (width 0.8128) (layer B.Cu) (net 7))
 (segment (start 25.4 35.56) (end 25.4 32.94) (width 0.8128) (layer B.Cu) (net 8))
 (segment (start 30.48 35.56) (end 30.48 32.94) (width 0.8128) (layer B.Cu) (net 9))
 (segment (start 35.56 35.56) (end 35.56 32.94) (width 0.8128) (layer B.Cu) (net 10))
 (segment (start 30.48 15.24) (end 30.48 12.7) (width 0.8128) (layer B.Cu) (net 11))
 (segment (start 30.48 12.7) (end 27.94 12.7) (width 0.8128) (layer B.Cu) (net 11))
 (segment (start 27.94 12.7) (end 27.94 10.16) (width 0.8128) (layer B.Cu) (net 11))
 (segment (start 38.1 15.24) (end 38.1 12.7) (width 0.8128) (layer B.Cu) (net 12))
 (segment (start 38.1 12.7) (end 35.56 12.7) (width 0.8128) (layer B.Cu) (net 12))
 (segment (start 35.56 12.7) (end 35.56 10.16) (width 0.8128) (layer B.Cu) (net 12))
 (segment (start 22.86 17.78) (end 22.86 20.32) (width 0.8128) (layer B.Cu) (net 13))
 (segment (start 22.86 17.78) (end 25.4 17.78) (width 0.8128) (layer B.Cu) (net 13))
 (segment (start 25.4 17.78) (end 25.4 15.24) (width 0.8128) (layer B.Cu) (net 13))
 (segment (start 25.4 15.24) (end 27.94 15.24) (width 0.8128) (layer B.Cu) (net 13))
 (segment (start 48.26 40.64) (end 53.34 40.64) (width 0.8128) (layer B.Cu) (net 14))
 (segment (start 53.34 40.64) (end 53.34 43.18) (width 0.8128) (layer B.Cu) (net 14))
 (segment (start 60.96 43.18) (end 55.88 43.18) (width 0.8128) (layer B.Cu) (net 15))
 (segment (start 55.88 48.26) (end 55.88 43.18) (width 0.8128) (layer B.Cu) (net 15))
 (segment (start 55.88 43.18) (end 55.88 40.64) (width 0.8128) (layer B.Cu) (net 15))
 (segment (start 27.94 22.86) (end 27.94 17.78) (width 0.8128) (layer B.Cu) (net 26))
 (segment (start 30.48 22.86) (end 30.48 17.78) (width 0.8128) (layer B.Cu) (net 27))
 (segment (start 30.48 17.78) (end 33.02 17.78) (width 0.8128) (layer B.Cu) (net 27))
 (segment (start 33.02 17.78) (end 33.02 15.24) (width 0.8128) (layer B.Cu) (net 27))
 (segment (start 33.02 15.24) (end 35.56 15.24) (width 0.8128) (layer B.Cu) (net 27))
 (segment (start 38.1 22.86) (end 38.1 17.78) (width 0.8128) (layer B.Cu) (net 28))
 (segment (start 35.56 22.86) (end 35.56 17.78) (width 0.8128) (layer B.Cu) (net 29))
 (segment (start 20.32 43.18) (end 20.32 38.1) (width 0.8128) (layer B.Cu) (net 16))
 (segment (start 30.48 48.26) (end 33.02 48.26) (width 0.8128) (layer B.Cu) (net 17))
 (segment (start 33.02 45.72) (end 33.02 48.26) (width 0.8128) (layer B.Cu) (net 17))
 (segment (start 33.02 48.26) (end 35.56 48.26) (width 0.8128) (layer B.Cu) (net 17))
 (segment (start 27.94 45.72) (end 27.94 48.26) (width 0.8128) (layer B.Cu) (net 17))
 (segment (start 25.4 48.26) (end 27.94 48.26) (width 0.8128) (layer B.Cu) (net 17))
 (segment (start 27.94 48.26) (end 30.48 48.26) (width 0.8128) (layer B.Cu) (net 17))
 (segment (start 20.32 48.26) (end 22.86 48.26) (width 0.8128) (layer B.Cu) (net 17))
 (segment (start 22.86 45.72) (end 22.86 48.26) (width 0.8128) (layer B.Cu) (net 17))
 (segment (start 22.86 48.26) (end 25.4 48.26) (width 0.8128) (layer B.Cu) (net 17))
 (segment (start 17.78 45.72) (end 17.78 48.26) (width 0.8128) (layer B.Cu) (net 17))
 (segment (start 12.7 48.26) (end 17.78 48.26) (width 0.8128) (layer B.Cu) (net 17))
 (segment (start 17.78 48.26) (end 20.32 48.26) (width 0.8128) (layer B.Cu) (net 17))
 (segment (start 33.02 45.72) (end 38.1 45.72) (width 0.8128) (layer B.Cu) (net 17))
 (segment (start 38.1 45.72) (end 38.1 38.1) (width 0.8128) (layer B.Cu) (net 17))
 (segment (start 38.1 38.1) (end 40.64 38.1) (width 0.8128) (layer B.Cu) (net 17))
 (segment (start 40.64 38.1) (end 40.64 35.56) (width 0.8128) (layer B.Cu) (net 17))
 (segment (start 25.4 43.18) (end 25.4 38.1) (width 0.8128) (layer B.Cu) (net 18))
 (segment (start 30.48 43.18) (end 30.48 38.1) (width 0.8128) (layer B.Cu) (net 19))
 (segment (start 35.56 43.18) (end 35.56 38.1) (width 0.8128) (layer B.Cu) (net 20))
 (segment (start 53.34 48.26) (end 48.26 48.26) (width 0.8128) (layer B.Cu) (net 22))
 (segment (start 40.64 45.72) (end 43.18 45.72) (width 0.8128) (layer F.Cu) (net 22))
 (segment (start 43.18 45.72) (end 45.72 48.26) (width 0.8128) (layer F.Cu) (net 22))
 (segment (start 45.72 48.26) (end 48.26 48.26) (width 0.8128) (layer F.Cu) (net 22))
 (segment (start 48.26 38.1) (end 53.34 38.1) (width 0.8128) (layer B.Cu) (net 25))
 (segment (start 40.64 40.64) (end 40.64 43.18) (width 0.8128) (layer B.Cu) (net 23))
 (segment (start 40.64 43.18) (end 43.18 43.18) (width 0.8128) (layer F.Cu) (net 23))
 (segment (start 45.72 45.72) (end 48.26 45.72) (width 0.8128) (layer F.Cu) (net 23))
 (segment (start 43.18 43.18) (end 45.72 45.72) (width 0.8128) (layer F.Cu) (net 23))
 (segment (start 48.26 35.56) (end 45.72 35.56) (width 0.8128) (layer B.Cu) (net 24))
 (segment (start 45.72 35.56) (end 45.72 43.18) (width 0.8128) (layer B.Cu) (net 24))
 (segment (start 45.72 43.18) (end 48.26 43.18) (width 0.8128) (layer B.Cu) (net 24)))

